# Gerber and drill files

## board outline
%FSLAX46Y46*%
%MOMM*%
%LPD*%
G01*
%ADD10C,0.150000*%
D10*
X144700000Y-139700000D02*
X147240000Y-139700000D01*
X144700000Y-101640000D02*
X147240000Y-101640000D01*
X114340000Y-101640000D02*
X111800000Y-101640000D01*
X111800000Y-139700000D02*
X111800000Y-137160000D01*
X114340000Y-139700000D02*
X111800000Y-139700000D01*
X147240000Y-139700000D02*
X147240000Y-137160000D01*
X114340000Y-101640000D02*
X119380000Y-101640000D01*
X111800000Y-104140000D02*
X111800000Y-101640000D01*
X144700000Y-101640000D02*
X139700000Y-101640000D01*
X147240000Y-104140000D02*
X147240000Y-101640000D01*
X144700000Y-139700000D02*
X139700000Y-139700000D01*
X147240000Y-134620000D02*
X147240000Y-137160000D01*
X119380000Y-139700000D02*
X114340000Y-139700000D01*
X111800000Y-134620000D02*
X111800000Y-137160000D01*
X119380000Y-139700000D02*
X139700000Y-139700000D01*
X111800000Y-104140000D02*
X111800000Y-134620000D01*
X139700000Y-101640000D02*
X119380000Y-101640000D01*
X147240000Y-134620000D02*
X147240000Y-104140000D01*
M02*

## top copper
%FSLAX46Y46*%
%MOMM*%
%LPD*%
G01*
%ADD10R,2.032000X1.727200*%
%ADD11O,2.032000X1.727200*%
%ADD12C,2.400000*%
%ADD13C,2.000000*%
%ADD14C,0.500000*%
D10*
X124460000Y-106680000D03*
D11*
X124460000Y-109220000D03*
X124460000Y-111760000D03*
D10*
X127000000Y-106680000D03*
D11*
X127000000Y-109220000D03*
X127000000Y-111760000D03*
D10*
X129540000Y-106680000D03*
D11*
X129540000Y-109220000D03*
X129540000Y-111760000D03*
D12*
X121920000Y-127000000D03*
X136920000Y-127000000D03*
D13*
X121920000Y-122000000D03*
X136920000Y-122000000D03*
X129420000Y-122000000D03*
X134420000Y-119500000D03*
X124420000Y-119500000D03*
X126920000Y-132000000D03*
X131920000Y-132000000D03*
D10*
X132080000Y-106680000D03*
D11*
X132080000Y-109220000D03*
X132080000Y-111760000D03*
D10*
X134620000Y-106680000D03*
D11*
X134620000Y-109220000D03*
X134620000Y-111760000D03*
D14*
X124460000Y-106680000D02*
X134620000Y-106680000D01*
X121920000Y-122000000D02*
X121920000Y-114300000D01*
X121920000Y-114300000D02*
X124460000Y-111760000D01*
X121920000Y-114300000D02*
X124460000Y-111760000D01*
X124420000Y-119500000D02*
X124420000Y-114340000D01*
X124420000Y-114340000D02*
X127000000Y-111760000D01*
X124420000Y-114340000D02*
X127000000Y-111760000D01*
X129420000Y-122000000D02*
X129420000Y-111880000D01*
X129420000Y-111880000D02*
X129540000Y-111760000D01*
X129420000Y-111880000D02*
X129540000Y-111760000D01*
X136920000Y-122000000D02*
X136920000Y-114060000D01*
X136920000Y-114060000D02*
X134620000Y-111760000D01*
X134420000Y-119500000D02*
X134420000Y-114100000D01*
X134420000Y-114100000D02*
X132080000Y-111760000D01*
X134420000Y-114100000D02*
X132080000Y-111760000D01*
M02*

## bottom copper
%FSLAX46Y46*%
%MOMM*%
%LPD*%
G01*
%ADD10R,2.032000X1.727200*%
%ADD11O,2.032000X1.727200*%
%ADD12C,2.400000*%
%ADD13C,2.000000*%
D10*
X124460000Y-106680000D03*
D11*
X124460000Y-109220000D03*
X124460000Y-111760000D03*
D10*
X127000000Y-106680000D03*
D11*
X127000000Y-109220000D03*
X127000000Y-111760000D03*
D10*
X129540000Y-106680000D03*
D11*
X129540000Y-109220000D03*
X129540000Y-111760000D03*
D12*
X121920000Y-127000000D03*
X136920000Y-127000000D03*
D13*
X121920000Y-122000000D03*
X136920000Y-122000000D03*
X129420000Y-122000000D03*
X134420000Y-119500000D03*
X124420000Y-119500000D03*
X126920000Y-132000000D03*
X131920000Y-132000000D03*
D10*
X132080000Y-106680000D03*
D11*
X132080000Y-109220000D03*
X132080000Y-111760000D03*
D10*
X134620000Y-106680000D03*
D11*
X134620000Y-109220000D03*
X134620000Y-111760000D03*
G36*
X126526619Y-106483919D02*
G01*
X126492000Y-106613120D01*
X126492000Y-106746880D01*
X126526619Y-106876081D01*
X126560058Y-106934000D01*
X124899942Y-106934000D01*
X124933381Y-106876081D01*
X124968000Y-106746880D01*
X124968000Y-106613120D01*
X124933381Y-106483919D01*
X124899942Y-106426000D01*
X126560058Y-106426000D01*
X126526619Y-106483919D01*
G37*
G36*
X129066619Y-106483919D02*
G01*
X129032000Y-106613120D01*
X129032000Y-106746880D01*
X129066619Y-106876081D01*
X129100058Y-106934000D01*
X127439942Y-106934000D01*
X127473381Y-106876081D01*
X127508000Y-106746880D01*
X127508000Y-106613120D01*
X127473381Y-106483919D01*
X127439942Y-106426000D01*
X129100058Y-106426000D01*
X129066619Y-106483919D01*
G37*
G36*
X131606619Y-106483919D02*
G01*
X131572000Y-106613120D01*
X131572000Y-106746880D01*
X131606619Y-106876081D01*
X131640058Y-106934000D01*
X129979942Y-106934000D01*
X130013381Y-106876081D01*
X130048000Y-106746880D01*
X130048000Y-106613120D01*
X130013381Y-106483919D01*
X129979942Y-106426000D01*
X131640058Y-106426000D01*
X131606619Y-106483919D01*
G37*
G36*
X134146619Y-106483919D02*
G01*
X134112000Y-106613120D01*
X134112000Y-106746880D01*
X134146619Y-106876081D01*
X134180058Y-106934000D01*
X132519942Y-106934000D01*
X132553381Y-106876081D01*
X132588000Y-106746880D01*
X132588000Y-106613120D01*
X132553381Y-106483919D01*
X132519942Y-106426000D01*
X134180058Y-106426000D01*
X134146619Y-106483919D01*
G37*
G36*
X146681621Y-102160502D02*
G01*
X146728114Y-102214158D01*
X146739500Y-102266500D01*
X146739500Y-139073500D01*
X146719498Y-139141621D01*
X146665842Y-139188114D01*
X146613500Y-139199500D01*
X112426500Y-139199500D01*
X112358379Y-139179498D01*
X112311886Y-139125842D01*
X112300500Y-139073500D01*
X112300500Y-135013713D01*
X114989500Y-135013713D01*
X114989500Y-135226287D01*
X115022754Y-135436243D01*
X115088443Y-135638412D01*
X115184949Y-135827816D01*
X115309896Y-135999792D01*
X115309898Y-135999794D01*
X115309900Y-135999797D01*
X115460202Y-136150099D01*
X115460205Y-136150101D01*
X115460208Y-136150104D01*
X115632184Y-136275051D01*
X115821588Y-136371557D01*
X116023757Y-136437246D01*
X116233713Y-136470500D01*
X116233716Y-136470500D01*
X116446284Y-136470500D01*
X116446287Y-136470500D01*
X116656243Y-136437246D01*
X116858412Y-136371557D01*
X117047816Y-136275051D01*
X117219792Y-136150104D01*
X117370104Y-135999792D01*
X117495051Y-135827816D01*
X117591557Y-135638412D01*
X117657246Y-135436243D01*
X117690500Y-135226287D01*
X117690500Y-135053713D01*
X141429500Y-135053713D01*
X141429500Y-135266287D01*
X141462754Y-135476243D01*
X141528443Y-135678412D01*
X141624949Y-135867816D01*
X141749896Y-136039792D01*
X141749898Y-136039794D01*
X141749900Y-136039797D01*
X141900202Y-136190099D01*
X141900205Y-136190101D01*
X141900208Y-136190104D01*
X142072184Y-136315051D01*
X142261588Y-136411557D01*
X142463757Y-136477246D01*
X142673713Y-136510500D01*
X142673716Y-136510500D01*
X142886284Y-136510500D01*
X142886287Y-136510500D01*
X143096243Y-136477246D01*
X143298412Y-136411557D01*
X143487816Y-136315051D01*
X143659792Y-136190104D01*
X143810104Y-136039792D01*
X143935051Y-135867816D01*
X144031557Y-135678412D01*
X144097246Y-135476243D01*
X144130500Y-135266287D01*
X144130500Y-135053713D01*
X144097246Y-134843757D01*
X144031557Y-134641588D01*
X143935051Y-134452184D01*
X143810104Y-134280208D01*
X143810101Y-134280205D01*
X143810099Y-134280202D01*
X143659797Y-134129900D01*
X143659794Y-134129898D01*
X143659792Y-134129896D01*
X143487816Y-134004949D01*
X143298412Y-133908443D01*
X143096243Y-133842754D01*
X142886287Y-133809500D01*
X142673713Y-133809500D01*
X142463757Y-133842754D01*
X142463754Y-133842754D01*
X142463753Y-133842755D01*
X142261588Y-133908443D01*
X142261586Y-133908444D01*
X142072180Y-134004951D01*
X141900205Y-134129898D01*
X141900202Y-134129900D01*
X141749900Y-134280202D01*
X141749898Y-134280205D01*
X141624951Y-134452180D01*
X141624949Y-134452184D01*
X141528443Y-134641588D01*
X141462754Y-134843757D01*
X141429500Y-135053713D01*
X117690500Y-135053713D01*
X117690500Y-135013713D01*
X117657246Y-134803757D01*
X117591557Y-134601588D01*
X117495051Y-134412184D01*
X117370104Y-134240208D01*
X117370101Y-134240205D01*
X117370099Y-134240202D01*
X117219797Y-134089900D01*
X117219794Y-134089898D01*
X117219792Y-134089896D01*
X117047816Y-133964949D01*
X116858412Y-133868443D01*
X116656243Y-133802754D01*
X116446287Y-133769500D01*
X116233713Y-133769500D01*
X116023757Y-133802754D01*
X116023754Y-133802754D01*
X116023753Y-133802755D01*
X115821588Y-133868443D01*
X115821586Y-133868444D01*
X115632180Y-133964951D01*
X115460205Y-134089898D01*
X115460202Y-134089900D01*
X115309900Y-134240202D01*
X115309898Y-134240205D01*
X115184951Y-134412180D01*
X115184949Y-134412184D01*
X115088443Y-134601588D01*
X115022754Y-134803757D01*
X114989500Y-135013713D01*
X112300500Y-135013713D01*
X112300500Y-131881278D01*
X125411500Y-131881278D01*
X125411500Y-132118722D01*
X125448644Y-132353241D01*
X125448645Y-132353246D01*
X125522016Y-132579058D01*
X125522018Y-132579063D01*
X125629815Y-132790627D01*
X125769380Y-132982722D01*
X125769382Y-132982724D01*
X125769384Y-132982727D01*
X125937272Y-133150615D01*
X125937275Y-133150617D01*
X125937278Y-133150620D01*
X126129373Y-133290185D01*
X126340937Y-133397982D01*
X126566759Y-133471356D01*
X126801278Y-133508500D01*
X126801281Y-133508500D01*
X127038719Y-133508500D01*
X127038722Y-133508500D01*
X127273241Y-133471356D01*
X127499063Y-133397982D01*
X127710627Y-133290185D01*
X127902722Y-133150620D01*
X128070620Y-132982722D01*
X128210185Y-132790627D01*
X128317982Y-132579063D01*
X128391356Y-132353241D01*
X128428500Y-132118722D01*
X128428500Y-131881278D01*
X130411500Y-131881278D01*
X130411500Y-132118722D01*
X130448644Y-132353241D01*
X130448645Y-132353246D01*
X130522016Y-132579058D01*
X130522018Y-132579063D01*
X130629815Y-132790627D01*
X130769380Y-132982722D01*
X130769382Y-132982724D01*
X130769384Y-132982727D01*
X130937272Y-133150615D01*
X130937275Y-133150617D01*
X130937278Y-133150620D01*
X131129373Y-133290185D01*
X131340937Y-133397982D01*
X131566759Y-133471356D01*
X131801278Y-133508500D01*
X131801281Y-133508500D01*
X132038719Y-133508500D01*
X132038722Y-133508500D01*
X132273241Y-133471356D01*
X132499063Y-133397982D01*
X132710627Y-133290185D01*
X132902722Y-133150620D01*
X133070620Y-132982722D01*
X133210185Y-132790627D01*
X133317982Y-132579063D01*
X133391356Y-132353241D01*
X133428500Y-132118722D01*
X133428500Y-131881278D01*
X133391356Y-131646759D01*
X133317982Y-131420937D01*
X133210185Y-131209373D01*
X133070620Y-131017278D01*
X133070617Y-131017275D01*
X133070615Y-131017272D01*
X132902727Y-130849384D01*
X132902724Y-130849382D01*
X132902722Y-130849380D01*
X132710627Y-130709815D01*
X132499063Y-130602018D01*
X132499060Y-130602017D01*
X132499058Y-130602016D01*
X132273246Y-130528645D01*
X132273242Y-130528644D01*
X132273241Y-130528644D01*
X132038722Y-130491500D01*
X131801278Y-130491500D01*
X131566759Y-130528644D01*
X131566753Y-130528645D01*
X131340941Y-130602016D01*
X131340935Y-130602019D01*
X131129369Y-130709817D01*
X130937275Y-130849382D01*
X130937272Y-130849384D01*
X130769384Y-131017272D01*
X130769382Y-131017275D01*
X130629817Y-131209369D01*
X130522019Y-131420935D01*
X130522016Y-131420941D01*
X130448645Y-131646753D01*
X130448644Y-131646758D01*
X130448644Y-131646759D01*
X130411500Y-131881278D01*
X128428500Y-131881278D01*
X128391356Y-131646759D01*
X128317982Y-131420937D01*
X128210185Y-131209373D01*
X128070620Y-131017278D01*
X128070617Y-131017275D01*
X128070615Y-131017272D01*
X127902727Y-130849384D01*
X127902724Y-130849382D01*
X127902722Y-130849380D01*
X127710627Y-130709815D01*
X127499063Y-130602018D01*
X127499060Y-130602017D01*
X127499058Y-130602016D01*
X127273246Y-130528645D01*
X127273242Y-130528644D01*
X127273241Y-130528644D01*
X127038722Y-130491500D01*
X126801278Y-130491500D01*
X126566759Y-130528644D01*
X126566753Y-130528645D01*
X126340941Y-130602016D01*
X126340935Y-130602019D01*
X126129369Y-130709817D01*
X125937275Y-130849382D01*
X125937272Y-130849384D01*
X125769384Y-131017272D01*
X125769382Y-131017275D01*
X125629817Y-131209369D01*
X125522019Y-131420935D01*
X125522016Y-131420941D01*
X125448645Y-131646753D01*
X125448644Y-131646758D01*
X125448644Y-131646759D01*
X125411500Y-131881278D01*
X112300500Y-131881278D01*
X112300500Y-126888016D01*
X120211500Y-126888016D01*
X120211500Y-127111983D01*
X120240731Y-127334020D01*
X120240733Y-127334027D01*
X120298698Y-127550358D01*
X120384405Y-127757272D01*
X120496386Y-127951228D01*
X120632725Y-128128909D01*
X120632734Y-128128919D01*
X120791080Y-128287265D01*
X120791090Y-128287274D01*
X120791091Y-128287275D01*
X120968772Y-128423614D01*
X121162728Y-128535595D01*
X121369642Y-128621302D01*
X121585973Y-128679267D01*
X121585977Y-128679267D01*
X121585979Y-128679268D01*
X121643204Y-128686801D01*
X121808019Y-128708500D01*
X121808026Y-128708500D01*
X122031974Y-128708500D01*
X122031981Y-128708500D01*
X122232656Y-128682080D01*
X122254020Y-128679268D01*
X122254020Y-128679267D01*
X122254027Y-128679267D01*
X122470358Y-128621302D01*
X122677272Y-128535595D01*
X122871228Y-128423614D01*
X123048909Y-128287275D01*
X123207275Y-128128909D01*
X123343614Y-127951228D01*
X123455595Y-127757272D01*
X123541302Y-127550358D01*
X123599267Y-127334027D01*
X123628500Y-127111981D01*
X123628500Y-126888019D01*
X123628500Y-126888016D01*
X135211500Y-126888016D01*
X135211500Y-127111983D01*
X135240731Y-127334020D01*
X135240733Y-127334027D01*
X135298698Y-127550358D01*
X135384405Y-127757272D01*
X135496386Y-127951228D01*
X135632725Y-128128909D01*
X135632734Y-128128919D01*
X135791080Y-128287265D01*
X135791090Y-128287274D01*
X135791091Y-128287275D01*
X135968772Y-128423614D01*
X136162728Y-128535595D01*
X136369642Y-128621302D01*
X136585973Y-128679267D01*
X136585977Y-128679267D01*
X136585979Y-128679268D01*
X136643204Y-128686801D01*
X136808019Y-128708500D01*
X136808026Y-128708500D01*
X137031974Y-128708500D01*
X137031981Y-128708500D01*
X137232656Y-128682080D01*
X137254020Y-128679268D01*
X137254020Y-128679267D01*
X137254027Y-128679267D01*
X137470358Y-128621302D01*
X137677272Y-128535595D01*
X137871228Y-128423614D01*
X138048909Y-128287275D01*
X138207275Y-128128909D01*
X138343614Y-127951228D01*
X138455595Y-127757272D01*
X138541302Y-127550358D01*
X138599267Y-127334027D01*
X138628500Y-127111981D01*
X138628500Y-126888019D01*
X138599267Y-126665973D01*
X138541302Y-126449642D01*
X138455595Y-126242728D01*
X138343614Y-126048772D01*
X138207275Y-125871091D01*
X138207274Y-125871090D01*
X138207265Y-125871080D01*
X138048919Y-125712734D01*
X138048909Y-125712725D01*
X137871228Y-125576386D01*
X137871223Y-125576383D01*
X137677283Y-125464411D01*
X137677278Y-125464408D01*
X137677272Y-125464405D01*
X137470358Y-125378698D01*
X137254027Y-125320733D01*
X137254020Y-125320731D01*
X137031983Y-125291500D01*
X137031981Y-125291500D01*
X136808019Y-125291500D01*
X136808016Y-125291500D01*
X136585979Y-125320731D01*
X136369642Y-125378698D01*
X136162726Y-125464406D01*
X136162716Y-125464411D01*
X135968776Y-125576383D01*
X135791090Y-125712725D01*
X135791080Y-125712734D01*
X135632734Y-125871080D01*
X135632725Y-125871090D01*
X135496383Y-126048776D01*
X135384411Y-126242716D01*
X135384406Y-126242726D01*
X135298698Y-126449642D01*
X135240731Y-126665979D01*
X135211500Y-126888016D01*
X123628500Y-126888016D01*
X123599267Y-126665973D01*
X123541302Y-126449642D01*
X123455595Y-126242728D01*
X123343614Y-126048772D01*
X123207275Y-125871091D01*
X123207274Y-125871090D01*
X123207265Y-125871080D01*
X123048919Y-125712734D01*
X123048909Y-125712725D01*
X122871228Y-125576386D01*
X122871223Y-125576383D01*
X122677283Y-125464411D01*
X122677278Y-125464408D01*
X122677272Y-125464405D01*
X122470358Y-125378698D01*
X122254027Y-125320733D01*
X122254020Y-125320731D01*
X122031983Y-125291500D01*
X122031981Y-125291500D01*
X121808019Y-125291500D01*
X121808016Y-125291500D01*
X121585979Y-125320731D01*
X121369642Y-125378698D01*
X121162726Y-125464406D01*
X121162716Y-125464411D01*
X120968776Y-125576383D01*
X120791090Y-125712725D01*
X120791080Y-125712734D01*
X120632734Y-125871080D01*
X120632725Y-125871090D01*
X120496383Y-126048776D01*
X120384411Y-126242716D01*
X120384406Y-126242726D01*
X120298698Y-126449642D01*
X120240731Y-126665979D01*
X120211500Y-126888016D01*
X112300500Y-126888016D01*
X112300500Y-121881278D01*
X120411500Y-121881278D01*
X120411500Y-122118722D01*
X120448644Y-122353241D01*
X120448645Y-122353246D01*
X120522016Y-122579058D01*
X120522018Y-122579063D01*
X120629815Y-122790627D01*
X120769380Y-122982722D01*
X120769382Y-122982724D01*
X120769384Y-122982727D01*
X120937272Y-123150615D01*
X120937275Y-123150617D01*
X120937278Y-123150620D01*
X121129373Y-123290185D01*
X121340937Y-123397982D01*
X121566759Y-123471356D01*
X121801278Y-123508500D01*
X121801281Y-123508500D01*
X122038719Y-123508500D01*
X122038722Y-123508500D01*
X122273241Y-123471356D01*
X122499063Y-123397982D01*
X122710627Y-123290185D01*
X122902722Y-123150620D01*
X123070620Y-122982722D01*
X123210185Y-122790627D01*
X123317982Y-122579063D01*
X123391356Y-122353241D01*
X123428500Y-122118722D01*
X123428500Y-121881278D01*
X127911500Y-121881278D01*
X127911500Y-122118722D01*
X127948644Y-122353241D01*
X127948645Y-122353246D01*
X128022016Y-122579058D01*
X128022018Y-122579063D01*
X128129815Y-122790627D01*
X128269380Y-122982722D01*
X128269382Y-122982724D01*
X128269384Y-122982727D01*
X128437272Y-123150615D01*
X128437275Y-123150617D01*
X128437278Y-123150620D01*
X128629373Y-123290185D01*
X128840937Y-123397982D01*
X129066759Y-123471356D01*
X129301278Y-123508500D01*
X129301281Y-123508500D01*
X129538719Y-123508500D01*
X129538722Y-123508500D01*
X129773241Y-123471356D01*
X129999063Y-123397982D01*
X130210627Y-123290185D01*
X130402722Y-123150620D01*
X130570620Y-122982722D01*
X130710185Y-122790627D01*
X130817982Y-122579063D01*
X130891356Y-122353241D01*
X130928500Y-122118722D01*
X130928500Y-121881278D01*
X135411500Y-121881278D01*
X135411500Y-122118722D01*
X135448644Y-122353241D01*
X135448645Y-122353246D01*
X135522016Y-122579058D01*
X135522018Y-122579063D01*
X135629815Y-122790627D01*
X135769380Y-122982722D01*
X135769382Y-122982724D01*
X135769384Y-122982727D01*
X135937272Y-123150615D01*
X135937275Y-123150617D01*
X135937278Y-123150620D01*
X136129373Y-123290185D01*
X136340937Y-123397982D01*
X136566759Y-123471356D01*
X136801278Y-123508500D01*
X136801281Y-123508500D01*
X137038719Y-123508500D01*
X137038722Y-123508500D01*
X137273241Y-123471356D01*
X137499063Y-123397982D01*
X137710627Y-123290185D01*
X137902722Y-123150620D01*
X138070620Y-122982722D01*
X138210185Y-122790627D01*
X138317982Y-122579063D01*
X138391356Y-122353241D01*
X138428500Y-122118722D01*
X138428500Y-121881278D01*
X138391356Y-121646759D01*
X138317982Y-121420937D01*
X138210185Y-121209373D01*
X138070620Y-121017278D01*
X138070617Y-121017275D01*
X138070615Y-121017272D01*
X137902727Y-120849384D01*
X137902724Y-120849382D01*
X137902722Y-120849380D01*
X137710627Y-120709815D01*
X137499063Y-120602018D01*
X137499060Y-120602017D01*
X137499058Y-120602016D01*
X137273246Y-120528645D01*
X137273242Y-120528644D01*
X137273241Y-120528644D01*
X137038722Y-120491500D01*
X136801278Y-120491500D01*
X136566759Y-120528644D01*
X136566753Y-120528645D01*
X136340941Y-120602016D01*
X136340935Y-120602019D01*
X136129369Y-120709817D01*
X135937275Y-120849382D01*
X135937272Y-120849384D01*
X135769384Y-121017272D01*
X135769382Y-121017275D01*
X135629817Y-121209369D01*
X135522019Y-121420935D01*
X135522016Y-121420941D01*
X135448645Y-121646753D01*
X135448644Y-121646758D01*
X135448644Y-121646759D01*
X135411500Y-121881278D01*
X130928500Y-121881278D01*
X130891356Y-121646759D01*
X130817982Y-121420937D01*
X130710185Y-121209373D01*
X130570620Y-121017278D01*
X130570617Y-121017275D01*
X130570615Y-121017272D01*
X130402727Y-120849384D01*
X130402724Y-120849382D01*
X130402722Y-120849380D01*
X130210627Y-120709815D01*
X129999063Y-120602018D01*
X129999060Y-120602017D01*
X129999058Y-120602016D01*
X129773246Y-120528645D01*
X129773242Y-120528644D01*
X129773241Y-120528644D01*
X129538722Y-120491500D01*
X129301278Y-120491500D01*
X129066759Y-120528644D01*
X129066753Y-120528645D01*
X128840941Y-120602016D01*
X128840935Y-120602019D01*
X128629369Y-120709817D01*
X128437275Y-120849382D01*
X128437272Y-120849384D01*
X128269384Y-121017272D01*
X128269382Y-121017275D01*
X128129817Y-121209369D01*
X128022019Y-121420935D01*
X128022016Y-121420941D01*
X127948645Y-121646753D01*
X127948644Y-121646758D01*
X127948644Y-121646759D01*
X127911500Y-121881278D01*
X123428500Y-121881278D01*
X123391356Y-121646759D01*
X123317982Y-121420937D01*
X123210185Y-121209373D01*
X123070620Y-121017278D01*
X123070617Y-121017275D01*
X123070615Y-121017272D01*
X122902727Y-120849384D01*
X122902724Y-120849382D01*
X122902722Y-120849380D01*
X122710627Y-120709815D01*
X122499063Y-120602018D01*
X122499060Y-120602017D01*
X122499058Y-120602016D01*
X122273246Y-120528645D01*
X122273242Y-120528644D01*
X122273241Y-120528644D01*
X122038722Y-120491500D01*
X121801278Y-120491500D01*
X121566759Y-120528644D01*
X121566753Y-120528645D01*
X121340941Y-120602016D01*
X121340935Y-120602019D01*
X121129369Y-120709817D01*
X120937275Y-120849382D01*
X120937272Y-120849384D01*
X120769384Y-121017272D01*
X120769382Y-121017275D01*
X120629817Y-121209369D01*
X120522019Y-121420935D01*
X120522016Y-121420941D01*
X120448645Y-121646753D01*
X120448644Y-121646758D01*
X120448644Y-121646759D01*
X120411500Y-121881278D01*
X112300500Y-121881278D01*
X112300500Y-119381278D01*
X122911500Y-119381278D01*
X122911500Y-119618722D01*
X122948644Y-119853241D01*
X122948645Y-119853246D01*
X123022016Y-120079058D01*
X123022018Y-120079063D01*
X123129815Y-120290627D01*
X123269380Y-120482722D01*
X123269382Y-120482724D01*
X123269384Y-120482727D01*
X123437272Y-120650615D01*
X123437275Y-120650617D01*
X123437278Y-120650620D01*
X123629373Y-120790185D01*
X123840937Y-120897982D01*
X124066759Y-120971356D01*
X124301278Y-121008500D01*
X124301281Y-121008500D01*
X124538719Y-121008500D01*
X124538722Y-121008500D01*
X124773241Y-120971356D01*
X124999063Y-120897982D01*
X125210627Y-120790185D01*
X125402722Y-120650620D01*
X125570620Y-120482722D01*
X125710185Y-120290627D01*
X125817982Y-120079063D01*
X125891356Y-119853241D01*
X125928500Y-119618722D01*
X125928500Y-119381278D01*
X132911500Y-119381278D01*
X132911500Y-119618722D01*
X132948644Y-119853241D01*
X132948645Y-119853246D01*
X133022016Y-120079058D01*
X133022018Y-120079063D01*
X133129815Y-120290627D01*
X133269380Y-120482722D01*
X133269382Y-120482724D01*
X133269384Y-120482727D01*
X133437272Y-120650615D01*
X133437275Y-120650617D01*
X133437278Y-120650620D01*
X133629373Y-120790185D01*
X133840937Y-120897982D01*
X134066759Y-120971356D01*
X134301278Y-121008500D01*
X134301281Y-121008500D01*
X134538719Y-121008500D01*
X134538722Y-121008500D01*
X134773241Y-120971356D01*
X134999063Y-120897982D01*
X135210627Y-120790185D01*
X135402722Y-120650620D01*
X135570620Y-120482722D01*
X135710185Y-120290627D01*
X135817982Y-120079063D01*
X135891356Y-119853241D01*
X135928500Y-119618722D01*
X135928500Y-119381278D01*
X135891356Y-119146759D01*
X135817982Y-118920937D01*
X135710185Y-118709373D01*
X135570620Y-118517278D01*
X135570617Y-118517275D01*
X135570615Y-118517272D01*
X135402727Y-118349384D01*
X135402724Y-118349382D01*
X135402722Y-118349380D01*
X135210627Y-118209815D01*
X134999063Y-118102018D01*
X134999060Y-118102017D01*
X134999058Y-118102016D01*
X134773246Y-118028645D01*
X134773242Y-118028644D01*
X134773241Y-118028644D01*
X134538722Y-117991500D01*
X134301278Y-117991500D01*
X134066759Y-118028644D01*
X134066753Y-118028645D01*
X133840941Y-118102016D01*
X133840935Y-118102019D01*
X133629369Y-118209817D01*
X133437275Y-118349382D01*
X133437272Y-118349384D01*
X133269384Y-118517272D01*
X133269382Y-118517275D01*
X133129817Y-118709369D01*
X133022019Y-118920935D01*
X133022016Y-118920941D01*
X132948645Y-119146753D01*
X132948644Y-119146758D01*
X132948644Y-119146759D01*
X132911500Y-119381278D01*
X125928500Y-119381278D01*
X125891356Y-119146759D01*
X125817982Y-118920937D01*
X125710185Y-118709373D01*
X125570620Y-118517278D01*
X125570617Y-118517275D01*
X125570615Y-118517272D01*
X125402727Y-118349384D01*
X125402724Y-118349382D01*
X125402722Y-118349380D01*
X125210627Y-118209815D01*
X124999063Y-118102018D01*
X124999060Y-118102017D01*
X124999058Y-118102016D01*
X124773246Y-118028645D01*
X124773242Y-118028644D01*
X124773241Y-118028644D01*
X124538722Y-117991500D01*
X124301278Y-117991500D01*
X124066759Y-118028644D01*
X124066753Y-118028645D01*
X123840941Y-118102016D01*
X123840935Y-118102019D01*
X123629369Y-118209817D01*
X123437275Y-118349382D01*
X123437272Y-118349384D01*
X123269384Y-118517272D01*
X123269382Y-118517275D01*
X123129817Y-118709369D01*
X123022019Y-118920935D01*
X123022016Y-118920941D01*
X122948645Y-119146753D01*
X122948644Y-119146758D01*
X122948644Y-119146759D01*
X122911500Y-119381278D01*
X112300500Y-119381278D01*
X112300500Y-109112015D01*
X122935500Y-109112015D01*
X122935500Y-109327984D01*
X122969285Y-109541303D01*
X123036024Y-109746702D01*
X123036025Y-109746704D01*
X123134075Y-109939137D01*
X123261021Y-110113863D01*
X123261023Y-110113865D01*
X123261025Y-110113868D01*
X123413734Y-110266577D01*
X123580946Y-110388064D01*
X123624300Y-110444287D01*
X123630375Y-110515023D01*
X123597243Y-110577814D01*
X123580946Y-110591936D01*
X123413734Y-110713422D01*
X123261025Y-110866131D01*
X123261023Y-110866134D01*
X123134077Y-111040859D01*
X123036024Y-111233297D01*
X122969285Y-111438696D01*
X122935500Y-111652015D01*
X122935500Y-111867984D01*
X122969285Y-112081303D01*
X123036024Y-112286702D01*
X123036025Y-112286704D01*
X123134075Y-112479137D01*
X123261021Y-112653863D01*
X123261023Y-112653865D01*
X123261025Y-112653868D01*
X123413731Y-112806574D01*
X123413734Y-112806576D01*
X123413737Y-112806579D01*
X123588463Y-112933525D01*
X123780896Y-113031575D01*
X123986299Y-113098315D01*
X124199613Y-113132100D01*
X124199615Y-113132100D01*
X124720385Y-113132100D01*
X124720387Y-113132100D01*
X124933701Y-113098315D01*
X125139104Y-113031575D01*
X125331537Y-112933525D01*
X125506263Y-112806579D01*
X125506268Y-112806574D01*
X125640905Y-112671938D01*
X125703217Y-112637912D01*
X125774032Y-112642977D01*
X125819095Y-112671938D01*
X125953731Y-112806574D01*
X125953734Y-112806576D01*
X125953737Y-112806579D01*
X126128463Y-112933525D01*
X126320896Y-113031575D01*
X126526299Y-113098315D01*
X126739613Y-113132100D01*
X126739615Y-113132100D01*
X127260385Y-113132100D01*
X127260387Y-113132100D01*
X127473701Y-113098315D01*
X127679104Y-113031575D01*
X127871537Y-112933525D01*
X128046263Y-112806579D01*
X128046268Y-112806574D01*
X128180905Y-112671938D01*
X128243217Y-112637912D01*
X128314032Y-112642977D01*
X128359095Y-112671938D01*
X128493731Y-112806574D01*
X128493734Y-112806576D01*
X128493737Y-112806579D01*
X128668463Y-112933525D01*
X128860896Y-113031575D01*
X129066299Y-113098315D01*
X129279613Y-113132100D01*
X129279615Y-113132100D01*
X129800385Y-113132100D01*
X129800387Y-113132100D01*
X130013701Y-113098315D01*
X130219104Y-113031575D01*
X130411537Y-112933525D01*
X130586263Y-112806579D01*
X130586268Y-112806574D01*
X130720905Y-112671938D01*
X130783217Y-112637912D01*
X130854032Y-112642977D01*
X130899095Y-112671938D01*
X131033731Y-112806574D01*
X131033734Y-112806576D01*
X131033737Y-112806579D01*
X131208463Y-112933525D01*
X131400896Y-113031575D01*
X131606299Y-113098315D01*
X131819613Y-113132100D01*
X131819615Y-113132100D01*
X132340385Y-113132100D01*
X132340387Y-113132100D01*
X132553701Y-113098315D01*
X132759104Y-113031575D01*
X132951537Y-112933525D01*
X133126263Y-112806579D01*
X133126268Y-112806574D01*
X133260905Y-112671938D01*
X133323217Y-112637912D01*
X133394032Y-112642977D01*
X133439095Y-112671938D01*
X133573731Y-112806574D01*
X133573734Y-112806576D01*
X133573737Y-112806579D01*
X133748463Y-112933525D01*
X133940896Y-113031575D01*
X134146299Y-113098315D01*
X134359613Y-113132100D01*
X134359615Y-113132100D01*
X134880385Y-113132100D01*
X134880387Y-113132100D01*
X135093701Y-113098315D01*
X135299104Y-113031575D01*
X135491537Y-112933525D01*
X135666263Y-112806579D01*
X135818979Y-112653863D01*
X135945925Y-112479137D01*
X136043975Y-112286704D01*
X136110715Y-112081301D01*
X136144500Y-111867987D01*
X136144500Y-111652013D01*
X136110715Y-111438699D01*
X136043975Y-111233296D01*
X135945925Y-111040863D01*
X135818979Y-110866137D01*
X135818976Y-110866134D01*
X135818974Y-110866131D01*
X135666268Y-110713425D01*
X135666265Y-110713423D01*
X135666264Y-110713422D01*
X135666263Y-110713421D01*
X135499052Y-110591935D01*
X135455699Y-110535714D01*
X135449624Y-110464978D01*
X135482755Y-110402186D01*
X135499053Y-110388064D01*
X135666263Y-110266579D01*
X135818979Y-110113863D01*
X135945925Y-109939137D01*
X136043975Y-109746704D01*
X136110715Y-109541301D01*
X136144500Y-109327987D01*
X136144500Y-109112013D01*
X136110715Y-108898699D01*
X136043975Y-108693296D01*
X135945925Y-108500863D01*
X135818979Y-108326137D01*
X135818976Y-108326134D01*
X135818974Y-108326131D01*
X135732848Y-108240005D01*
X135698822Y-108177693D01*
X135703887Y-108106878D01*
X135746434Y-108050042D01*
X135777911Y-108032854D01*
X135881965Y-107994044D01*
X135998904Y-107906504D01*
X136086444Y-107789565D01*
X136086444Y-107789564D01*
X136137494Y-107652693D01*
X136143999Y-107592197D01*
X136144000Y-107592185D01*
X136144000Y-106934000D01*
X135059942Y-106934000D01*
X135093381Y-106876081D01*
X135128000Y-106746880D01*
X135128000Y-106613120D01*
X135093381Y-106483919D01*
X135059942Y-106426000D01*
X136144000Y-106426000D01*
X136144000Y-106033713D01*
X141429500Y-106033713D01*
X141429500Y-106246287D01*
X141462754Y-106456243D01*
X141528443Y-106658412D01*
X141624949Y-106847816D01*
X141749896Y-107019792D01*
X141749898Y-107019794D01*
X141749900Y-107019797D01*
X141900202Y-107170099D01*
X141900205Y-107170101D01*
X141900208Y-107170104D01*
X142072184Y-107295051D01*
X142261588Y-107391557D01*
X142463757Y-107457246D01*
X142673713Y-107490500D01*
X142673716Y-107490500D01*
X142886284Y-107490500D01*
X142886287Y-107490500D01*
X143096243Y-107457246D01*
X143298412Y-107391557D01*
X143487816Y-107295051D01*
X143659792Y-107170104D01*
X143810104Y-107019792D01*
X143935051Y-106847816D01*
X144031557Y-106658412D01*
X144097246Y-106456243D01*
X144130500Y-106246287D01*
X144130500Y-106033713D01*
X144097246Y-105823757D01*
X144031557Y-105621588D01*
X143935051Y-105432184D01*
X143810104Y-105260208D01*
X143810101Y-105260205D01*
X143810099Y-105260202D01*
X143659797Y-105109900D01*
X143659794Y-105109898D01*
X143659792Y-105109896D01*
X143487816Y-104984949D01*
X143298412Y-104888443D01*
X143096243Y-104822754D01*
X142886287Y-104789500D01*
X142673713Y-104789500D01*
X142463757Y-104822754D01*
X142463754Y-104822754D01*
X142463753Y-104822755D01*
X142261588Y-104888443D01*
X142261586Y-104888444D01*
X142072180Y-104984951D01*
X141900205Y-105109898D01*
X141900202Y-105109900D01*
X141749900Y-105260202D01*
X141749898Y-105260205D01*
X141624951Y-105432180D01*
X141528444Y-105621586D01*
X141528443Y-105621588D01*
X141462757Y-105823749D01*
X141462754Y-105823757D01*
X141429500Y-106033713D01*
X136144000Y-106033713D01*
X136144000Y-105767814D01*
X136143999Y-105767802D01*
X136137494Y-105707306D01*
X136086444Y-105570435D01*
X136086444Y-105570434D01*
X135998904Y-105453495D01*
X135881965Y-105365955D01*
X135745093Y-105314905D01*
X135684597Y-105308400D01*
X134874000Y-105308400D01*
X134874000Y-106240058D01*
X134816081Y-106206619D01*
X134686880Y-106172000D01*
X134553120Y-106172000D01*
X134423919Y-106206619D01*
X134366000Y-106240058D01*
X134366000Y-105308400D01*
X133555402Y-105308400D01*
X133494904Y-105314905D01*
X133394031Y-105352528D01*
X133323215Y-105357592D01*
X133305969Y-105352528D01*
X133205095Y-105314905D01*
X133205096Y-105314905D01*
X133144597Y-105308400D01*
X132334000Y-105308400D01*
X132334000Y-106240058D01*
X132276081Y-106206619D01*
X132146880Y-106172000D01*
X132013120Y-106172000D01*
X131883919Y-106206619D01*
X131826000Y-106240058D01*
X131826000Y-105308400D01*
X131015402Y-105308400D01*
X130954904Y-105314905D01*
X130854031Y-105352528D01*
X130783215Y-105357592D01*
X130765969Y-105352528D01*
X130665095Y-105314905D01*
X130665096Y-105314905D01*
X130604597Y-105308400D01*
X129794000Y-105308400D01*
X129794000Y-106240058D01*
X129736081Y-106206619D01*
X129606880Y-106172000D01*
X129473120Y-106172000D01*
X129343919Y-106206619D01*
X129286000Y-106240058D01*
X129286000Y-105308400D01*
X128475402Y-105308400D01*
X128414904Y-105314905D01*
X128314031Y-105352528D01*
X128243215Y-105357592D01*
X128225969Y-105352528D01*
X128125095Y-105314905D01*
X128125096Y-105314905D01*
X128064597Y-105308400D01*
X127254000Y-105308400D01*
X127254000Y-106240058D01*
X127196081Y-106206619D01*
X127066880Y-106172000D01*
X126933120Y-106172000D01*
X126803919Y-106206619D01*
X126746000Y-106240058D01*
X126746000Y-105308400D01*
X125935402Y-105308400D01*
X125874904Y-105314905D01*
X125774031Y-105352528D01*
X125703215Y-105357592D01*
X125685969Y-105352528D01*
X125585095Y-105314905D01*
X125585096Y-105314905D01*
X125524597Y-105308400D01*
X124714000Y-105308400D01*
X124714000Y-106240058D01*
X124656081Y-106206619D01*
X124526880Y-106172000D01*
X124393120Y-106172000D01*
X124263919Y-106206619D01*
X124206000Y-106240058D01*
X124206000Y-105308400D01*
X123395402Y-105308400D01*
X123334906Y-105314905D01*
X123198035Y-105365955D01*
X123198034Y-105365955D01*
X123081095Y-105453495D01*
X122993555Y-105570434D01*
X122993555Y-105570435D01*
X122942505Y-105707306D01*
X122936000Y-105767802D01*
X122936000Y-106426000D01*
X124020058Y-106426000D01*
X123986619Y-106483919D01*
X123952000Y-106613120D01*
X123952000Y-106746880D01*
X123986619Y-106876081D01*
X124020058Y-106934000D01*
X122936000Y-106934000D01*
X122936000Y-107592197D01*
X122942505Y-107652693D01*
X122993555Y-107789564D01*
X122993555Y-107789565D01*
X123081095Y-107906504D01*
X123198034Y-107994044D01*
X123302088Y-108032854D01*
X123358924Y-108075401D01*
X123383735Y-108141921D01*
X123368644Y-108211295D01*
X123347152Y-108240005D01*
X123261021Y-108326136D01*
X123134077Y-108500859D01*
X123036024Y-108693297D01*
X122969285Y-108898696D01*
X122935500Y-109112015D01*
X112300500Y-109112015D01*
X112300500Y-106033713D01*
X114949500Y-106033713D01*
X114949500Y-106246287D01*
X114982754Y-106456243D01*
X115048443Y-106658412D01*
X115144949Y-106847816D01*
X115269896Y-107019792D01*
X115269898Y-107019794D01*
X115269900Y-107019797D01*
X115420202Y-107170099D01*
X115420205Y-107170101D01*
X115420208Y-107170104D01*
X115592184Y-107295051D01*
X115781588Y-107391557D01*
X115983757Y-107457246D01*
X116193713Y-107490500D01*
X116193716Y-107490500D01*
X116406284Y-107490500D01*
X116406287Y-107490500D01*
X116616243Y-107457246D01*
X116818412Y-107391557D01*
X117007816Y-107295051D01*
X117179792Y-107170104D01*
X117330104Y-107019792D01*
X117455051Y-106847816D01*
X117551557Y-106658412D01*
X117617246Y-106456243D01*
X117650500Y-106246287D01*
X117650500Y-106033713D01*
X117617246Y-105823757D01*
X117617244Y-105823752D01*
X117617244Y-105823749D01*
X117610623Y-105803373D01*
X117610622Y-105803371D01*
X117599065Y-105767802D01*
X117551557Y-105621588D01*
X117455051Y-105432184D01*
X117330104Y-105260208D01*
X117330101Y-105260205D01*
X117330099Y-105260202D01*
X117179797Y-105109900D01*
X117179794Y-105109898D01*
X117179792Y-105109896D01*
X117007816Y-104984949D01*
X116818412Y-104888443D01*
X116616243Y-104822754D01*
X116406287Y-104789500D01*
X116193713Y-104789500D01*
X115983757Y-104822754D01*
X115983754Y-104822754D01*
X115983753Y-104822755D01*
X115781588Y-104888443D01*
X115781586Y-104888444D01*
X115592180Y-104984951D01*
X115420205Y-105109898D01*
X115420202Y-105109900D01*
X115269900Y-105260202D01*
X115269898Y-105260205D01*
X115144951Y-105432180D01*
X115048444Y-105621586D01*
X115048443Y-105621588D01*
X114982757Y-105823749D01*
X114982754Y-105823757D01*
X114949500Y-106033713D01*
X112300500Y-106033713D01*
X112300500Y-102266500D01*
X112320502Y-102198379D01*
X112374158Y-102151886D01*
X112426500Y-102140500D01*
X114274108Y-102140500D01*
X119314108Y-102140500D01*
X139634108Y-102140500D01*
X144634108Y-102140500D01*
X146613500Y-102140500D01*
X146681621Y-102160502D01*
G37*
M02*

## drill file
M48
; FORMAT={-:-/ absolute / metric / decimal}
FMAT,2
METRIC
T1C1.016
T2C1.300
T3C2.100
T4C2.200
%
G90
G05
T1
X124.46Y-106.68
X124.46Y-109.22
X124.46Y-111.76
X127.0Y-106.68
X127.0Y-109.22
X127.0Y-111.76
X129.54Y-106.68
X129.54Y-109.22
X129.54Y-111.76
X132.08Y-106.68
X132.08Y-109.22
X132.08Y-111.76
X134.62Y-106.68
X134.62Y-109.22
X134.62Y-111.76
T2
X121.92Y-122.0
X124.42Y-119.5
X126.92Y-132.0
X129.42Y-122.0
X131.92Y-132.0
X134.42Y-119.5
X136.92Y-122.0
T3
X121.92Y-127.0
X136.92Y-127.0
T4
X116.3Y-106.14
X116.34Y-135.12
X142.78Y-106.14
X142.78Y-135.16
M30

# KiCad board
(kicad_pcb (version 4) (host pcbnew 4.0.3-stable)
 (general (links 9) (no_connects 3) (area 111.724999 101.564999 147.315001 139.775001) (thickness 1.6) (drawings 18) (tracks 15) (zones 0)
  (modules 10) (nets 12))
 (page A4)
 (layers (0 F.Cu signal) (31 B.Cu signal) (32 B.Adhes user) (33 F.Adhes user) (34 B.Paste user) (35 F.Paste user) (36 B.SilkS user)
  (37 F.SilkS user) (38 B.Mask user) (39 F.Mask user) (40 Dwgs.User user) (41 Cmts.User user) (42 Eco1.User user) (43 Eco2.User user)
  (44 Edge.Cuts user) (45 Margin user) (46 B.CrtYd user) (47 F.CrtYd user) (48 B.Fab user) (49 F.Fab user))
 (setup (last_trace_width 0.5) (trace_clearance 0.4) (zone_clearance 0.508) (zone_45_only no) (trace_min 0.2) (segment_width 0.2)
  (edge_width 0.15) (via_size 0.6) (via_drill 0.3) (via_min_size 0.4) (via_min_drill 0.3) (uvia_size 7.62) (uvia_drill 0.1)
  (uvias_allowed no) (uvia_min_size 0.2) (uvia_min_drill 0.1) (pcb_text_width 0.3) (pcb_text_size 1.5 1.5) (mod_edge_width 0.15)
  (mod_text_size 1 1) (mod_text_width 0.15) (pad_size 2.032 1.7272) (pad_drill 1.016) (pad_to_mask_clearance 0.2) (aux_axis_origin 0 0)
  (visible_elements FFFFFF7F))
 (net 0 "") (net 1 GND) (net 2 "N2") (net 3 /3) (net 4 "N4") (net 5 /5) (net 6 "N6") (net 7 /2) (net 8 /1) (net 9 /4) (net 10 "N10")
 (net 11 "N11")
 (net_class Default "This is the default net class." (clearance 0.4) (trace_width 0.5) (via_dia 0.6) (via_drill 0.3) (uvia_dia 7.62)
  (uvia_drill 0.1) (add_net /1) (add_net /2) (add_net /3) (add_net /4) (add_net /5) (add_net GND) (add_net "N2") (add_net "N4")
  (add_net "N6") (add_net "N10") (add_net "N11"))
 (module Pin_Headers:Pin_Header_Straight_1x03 (layer F.Cu) (at 124.46 106.68)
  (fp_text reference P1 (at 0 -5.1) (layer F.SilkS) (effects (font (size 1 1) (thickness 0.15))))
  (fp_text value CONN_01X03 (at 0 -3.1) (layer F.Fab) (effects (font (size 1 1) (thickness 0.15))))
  (pad 1 thru_hole rect (at 0 0) (size 2.032 1.7272) (drill 1.016) (layers *.Cu *.Mask F.SilkS) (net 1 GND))
  (pad 2 thru_hole oval (at 0 2.54) (size 2.032 1.7272) (drill 1.016) (layers *.Cu *.Mask F.SilkS) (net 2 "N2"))
  (pad 3 thru_hole oval (at 0 5.08) (size 2.032 1.7272) (drill 1.016) (layers *.Cu *.Mask F.SilkS) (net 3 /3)))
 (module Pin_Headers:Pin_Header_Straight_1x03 (layer F.Cu) (at 127 106.68)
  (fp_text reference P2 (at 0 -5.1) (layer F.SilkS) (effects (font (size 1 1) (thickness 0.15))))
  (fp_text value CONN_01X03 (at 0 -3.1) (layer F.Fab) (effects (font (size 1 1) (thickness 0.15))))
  (pad 1 thru_hole rect (at 0 0) (size 2.032 1.7272) (drill 1.016) (layers *.Cu *.Mask F.SilkS) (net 1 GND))
  (pad 2 thru_hole oval (at 0 2.54) (size 2.032 1.7272) (drill 1.016) (layers *.Cu *.Mask F.SilkS) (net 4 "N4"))
  (pad 3 thru_hole oval (at 0 5.08) (size 2.032 1.7272) (drill 1.016) (layers *.Cu *.Mask F.SilkS) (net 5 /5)))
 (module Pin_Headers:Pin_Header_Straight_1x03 (layer F.Cu) (at 129.54 106.68)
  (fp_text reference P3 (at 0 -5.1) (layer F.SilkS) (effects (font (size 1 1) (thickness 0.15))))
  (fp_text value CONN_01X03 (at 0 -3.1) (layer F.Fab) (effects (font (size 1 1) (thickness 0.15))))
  (pad 1 thru_hole rect (at 0 0) (size 2.032 1.7272) (drill 1.016) (layers *.Cu *.Mask F.SilkS) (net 1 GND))
  (pad 2 thru_hole oval (at 0 2.54) (size 2.032 1.7272) (drill 1.016) (layers *.Cu *.Mask F.SilkS) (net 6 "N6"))
  (pad 3 thru_hole oval (at 0 5.08) (size 2.032 1.7272) (drill 1.016) (layers *.Cu *.Mask F.SilkS) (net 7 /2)))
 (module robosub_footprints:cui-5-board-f (layer F.Cu) (at 121.92 127)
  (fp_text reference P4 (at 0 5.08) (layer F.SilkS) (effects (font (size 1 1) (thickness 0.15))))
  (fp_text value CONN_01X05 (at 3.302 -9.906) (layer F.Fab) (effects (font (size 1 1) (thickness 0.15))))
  (pad ~ thru_hole circle (at 0 0) (size 2.4 2.4) (drill 2.1) (layers *.Cu *.Mask F.SilkS))
  (pad ~ thru_hole circle (at 15 0) (size 2.4 2.4) (drill 2.1) (layers *.Cu *.Mask F.SilkS))
  (pad 3 thru_hole circle (at 0 -5) (size 2 2) (drill 1.3) (layers *.Cu *.Mask F.SilkS) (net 3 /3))
  (pad 1 thru_hole circle (at 15 -5) (size 2 2) (drill 1.3) (layers *.Cu *.Mask F.SilkS) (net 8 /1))
  (pad 2 thru_hole circle (at 7.5 -5) (size 2 2) (drill 1.3) (layers *.Cu *.Mask F.SilkS) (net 7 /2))
  (pad 4 thru_hole circle (at 12.5 -7.5) (size 2 2) (drill 1.3) (layers *.Cu *.Mask F.SilkS) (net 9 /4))
  (pad 5 thru_hole circle (at 2.5 -7.5) (size 2 2) (drill 1.3) (layers *.Cu *.Mask F.SilkS) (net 5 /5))
  (pad ~ thru_hole circle (at 5 5) (size 2 2) (drill 1.3) (layers *.Cu *.Mask F.SilkS))
  (pad ~ thru_hole circle (at 10 5) (size 2 2) (drill 1.3) (layers *.Cu *.Mask F.SilkS)))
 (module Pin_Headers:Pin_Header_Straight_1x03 (layer F.Cu) (at 132.08 106.68)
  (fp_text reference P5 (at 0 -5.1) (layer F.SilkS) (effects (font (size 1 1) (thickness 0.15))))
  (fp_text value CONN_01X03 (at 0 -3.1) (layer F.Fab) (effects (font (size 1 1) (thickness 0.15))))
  (pad 1 thru_hole rect (at 0 0) (size 2.032 1.7272) (drill 1.016) (layers *.Cu *.Mask F.SilkS) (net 1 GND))
  (pad 2 thru_hole oval (at 0 2.54) (size 2.032 1.7272) (drill 1.016) (layers *.Cu *.Mask F.SilkS) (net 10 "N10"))
  (pad 3 thru_hole oval (at 0 5.08) (size 2.032 1.7272) (drill 1.016) (layers *.Cu *.Mask F.SilkS) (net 9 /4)))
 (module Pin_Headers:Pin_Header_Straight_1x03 (layer F.Cu) (at 134.62 106.68)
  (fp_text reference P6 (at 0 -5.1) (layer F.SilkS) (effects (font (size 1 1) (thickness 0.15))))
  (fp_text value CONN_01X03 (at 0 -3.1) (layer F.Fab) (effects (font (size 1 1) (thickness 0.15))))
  (pad 1 thru_hole rect (at 0 0) (size 2.032 1.7272) (drill 1.016) (layers *.Cu *.Mask F.SilkS) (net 1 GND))
  (pad 2 thru_hole oval (at 0 2.54) (size 2.032 1.7272) (drill 1.016) (layers *.Cu *.Mask F.SilkS) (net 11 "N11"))
  (pad 3 thru_hole oval (at 0 5.08) (size 2.032 1.7272) (drill 1.016) (layers *.Cu *.Mask F.SilkS) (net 8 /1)))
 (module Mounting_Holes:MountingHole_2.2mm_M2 (layer F.Cu) (at 142.78 106.14)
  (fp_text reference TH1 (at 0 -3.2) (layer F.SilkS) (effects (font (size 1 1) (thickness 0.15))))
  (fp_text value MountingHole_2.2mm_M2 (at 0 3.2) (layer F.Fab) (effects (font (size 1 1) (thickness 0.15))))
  (pad 1 np_thru_hole circle (at 0 0) (size 2.2 2.2) (drill 2.2) (layers *.Cu *.Mask F.SilkS)))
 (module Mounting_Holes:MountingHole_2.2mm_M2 (layer F.Cu) (at 116.34 135.12)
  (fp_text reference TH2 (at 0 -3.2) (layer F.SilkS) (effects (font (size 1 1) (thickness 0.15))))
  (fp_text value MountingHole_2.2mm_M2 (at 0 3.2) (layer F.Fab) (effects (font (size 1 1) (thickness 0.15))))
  (pad 1 np_thru_hole circle (at 0 0) (size 2.2 2.2) (drill 2.2) (layers *.Cu *.Mask F.SilkS)))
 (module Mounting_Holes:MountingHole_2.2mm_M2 (layer F.Cu) (at 116.3 106.14)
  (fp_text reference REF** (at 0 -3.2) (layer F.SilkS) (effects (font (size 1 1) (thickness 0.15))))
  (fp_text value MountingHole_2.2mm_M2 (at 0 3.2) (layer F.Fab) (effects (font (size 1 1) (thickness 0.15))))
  (pad 1 np_thru_hole circle (at 0 0) (size 2.2 2.2) (drill 2.2) (layers *.Cu *.Mask F.SilkS)))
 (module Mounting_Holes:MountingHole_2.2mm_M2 (layer F.Cu) (at 142.78 135.16)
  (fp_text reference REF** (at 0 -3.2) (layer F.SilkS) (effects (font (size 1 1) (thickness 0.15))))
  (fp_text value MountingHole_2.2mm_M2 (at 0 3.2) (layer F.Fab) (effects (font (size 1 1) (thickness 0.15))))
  (pad 1 np_thru_hole circle (at 0 0) (size 2.2 2.2) (drill 2.2) (layers *.Cu *.Mask F.SilkS)))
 (gr_line (start 144.7 139.7) (end 147.24 139.7) (angle 90) (layer Edge.Cuts) (width 0.15))
 (gr_line (start 144.7 101.64) (end 147.24 101.64) (angle 90) (layer Edge.Cuts) (width 0.15))
 (gr_line (start 114.34 101.64) (end 111.8 101.64) (angle 90) (layer Edge.Cuts) (width 0.15))
 (gr_line (start 111.8 139.7) (end 111.8 137.16) (angle 90) (layer Edge.Cuts) (width 0.15))
 (gr_line (start 114.34 139.7) (end 111.8 139.7) (angle 90) (layer Edge.Cuts) (width 0.15))
 (gr_line (start 147.24 139.7) (end 147.24 137.16) (angle 90) (layer Edge.Cuts) (width 0.15))
 (gr_line (start 114.34 101.64) (end 119.38 101.64) (angle 90) (layer Edge.Cuts) (width 0.15))
 (gr_line (start 111.8 104.14) (end 111.8 101.64) (angle 90) (layer Edge.Cuts) (width 0.15))
 (gr_line (start 144.7 101.64) (end 139.7 101.64) (angle 90) (layer Edge.Cuts) (width 0.15))
 (gr_line (start 147.24 104.14) (end 147.24 101.64) (angle 90) (layer Edge.Cuts) (width 0.15))
 (gr_line (start 144.7 139.7) (end 139.7 139.7) (angle 90) (layer Edge.Cuts) (width 0.15))
 (gr_line (start 147.24 134.62) (end 147.24 137.16) (angle 90) (layer Edge.Cuts) (width 0.15))
 (gr_line (start 119.38 139.7) (end 114.34 139.7) (angle 90) (layer Edge.Cuts) (width 0.15))
 (gr_line (start 111.8 134.62) (end 111.8 137.16) (angle 90) (layer Edge.Cuts) (width 0.15))
 (gr_line (start 119.38 139.7) (end 139.7 139.7) (angle 90) (layer Edge.Cuts) (width 0.15))
 (gr_line (start 111.8 104.14) (end 111.8 134.62) (angle 90) (layer Edge.Cuts) (width 0.15))
 (gr_line (start 139.7 101.64) (end 119.38 101.64) (angle 90) (layer Edge.Cuts) (width 0.15))
 (gr_line (start 147.24 134.62) (end 147.24 104.14) (angle 90) (layer Edge.Cuts) (width 0.15))
 (segment (start 124.46 106.68) (end 134.62 106.68) (width 0.5) (layer F.Cu) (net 1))
 (segment (start 121.92 122) (end 121.92 114.3) (width 0.5) (layer F.Cu) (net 3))
 (segment (start 121.92 114.3) (end 124.46 111.76) (width 0.5) (layer F.Cu) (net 3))
 (segment (start 121.92 114.3) (end 124.46 111.76) (width 0.5) (layer F.Cu) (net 3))
 (segment (start 124.42 119.5) (end 124.42 114.34) (width 0.5) (layer F.Cu) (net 5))
 (segment (start 124.42 114.34) (end 127 111.76) (width 0.5) (layer F.Cu) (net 5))
 (segment (start 124.42 114.34) (end 127 111.76) (width 0.5) (layer F.Cu) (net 5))
 (segment (start 129.42 122) (end 129.42 111.88) (width 0.5) (layer F.Cu) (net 7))
 (segment (start 129.42 111.88) (end 129.54 111.76) (width 0.5) (layer F.Cu) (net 7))
 (segment (start 129.42 111.88) (end 129.54 111.76) (width 0.5) (layer F.Cu) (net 7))
 (segment (start 136.92 122) (end 136.92 114.06) (width 0.5) (layer F.Cu) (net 8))
 (segment (start 136.92 114.06) (end 134.62 111.76) (width 0.5) (layer F.Cu) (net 8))
 (segment (start 134.42 119.5) (end 134.42 114.1) (width 0.5) (layer F.Cu) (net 9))
 (segment (start 134.42 114.1) (end 132.08 111.76) (width 0.5) (layer F.Cu) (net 9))
 (segment (start 134.42 114.1) (end 132.08 111.76) (width 0.5) (layer F.Cu) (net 9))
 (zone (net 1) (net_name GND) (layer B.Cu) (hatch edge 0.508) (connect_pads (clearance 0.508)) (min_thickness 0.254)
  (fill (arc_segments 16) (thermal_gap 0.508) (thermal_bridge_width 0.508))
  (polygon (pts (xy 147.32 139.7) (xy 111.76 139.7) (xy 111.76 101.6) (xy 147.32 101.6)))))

